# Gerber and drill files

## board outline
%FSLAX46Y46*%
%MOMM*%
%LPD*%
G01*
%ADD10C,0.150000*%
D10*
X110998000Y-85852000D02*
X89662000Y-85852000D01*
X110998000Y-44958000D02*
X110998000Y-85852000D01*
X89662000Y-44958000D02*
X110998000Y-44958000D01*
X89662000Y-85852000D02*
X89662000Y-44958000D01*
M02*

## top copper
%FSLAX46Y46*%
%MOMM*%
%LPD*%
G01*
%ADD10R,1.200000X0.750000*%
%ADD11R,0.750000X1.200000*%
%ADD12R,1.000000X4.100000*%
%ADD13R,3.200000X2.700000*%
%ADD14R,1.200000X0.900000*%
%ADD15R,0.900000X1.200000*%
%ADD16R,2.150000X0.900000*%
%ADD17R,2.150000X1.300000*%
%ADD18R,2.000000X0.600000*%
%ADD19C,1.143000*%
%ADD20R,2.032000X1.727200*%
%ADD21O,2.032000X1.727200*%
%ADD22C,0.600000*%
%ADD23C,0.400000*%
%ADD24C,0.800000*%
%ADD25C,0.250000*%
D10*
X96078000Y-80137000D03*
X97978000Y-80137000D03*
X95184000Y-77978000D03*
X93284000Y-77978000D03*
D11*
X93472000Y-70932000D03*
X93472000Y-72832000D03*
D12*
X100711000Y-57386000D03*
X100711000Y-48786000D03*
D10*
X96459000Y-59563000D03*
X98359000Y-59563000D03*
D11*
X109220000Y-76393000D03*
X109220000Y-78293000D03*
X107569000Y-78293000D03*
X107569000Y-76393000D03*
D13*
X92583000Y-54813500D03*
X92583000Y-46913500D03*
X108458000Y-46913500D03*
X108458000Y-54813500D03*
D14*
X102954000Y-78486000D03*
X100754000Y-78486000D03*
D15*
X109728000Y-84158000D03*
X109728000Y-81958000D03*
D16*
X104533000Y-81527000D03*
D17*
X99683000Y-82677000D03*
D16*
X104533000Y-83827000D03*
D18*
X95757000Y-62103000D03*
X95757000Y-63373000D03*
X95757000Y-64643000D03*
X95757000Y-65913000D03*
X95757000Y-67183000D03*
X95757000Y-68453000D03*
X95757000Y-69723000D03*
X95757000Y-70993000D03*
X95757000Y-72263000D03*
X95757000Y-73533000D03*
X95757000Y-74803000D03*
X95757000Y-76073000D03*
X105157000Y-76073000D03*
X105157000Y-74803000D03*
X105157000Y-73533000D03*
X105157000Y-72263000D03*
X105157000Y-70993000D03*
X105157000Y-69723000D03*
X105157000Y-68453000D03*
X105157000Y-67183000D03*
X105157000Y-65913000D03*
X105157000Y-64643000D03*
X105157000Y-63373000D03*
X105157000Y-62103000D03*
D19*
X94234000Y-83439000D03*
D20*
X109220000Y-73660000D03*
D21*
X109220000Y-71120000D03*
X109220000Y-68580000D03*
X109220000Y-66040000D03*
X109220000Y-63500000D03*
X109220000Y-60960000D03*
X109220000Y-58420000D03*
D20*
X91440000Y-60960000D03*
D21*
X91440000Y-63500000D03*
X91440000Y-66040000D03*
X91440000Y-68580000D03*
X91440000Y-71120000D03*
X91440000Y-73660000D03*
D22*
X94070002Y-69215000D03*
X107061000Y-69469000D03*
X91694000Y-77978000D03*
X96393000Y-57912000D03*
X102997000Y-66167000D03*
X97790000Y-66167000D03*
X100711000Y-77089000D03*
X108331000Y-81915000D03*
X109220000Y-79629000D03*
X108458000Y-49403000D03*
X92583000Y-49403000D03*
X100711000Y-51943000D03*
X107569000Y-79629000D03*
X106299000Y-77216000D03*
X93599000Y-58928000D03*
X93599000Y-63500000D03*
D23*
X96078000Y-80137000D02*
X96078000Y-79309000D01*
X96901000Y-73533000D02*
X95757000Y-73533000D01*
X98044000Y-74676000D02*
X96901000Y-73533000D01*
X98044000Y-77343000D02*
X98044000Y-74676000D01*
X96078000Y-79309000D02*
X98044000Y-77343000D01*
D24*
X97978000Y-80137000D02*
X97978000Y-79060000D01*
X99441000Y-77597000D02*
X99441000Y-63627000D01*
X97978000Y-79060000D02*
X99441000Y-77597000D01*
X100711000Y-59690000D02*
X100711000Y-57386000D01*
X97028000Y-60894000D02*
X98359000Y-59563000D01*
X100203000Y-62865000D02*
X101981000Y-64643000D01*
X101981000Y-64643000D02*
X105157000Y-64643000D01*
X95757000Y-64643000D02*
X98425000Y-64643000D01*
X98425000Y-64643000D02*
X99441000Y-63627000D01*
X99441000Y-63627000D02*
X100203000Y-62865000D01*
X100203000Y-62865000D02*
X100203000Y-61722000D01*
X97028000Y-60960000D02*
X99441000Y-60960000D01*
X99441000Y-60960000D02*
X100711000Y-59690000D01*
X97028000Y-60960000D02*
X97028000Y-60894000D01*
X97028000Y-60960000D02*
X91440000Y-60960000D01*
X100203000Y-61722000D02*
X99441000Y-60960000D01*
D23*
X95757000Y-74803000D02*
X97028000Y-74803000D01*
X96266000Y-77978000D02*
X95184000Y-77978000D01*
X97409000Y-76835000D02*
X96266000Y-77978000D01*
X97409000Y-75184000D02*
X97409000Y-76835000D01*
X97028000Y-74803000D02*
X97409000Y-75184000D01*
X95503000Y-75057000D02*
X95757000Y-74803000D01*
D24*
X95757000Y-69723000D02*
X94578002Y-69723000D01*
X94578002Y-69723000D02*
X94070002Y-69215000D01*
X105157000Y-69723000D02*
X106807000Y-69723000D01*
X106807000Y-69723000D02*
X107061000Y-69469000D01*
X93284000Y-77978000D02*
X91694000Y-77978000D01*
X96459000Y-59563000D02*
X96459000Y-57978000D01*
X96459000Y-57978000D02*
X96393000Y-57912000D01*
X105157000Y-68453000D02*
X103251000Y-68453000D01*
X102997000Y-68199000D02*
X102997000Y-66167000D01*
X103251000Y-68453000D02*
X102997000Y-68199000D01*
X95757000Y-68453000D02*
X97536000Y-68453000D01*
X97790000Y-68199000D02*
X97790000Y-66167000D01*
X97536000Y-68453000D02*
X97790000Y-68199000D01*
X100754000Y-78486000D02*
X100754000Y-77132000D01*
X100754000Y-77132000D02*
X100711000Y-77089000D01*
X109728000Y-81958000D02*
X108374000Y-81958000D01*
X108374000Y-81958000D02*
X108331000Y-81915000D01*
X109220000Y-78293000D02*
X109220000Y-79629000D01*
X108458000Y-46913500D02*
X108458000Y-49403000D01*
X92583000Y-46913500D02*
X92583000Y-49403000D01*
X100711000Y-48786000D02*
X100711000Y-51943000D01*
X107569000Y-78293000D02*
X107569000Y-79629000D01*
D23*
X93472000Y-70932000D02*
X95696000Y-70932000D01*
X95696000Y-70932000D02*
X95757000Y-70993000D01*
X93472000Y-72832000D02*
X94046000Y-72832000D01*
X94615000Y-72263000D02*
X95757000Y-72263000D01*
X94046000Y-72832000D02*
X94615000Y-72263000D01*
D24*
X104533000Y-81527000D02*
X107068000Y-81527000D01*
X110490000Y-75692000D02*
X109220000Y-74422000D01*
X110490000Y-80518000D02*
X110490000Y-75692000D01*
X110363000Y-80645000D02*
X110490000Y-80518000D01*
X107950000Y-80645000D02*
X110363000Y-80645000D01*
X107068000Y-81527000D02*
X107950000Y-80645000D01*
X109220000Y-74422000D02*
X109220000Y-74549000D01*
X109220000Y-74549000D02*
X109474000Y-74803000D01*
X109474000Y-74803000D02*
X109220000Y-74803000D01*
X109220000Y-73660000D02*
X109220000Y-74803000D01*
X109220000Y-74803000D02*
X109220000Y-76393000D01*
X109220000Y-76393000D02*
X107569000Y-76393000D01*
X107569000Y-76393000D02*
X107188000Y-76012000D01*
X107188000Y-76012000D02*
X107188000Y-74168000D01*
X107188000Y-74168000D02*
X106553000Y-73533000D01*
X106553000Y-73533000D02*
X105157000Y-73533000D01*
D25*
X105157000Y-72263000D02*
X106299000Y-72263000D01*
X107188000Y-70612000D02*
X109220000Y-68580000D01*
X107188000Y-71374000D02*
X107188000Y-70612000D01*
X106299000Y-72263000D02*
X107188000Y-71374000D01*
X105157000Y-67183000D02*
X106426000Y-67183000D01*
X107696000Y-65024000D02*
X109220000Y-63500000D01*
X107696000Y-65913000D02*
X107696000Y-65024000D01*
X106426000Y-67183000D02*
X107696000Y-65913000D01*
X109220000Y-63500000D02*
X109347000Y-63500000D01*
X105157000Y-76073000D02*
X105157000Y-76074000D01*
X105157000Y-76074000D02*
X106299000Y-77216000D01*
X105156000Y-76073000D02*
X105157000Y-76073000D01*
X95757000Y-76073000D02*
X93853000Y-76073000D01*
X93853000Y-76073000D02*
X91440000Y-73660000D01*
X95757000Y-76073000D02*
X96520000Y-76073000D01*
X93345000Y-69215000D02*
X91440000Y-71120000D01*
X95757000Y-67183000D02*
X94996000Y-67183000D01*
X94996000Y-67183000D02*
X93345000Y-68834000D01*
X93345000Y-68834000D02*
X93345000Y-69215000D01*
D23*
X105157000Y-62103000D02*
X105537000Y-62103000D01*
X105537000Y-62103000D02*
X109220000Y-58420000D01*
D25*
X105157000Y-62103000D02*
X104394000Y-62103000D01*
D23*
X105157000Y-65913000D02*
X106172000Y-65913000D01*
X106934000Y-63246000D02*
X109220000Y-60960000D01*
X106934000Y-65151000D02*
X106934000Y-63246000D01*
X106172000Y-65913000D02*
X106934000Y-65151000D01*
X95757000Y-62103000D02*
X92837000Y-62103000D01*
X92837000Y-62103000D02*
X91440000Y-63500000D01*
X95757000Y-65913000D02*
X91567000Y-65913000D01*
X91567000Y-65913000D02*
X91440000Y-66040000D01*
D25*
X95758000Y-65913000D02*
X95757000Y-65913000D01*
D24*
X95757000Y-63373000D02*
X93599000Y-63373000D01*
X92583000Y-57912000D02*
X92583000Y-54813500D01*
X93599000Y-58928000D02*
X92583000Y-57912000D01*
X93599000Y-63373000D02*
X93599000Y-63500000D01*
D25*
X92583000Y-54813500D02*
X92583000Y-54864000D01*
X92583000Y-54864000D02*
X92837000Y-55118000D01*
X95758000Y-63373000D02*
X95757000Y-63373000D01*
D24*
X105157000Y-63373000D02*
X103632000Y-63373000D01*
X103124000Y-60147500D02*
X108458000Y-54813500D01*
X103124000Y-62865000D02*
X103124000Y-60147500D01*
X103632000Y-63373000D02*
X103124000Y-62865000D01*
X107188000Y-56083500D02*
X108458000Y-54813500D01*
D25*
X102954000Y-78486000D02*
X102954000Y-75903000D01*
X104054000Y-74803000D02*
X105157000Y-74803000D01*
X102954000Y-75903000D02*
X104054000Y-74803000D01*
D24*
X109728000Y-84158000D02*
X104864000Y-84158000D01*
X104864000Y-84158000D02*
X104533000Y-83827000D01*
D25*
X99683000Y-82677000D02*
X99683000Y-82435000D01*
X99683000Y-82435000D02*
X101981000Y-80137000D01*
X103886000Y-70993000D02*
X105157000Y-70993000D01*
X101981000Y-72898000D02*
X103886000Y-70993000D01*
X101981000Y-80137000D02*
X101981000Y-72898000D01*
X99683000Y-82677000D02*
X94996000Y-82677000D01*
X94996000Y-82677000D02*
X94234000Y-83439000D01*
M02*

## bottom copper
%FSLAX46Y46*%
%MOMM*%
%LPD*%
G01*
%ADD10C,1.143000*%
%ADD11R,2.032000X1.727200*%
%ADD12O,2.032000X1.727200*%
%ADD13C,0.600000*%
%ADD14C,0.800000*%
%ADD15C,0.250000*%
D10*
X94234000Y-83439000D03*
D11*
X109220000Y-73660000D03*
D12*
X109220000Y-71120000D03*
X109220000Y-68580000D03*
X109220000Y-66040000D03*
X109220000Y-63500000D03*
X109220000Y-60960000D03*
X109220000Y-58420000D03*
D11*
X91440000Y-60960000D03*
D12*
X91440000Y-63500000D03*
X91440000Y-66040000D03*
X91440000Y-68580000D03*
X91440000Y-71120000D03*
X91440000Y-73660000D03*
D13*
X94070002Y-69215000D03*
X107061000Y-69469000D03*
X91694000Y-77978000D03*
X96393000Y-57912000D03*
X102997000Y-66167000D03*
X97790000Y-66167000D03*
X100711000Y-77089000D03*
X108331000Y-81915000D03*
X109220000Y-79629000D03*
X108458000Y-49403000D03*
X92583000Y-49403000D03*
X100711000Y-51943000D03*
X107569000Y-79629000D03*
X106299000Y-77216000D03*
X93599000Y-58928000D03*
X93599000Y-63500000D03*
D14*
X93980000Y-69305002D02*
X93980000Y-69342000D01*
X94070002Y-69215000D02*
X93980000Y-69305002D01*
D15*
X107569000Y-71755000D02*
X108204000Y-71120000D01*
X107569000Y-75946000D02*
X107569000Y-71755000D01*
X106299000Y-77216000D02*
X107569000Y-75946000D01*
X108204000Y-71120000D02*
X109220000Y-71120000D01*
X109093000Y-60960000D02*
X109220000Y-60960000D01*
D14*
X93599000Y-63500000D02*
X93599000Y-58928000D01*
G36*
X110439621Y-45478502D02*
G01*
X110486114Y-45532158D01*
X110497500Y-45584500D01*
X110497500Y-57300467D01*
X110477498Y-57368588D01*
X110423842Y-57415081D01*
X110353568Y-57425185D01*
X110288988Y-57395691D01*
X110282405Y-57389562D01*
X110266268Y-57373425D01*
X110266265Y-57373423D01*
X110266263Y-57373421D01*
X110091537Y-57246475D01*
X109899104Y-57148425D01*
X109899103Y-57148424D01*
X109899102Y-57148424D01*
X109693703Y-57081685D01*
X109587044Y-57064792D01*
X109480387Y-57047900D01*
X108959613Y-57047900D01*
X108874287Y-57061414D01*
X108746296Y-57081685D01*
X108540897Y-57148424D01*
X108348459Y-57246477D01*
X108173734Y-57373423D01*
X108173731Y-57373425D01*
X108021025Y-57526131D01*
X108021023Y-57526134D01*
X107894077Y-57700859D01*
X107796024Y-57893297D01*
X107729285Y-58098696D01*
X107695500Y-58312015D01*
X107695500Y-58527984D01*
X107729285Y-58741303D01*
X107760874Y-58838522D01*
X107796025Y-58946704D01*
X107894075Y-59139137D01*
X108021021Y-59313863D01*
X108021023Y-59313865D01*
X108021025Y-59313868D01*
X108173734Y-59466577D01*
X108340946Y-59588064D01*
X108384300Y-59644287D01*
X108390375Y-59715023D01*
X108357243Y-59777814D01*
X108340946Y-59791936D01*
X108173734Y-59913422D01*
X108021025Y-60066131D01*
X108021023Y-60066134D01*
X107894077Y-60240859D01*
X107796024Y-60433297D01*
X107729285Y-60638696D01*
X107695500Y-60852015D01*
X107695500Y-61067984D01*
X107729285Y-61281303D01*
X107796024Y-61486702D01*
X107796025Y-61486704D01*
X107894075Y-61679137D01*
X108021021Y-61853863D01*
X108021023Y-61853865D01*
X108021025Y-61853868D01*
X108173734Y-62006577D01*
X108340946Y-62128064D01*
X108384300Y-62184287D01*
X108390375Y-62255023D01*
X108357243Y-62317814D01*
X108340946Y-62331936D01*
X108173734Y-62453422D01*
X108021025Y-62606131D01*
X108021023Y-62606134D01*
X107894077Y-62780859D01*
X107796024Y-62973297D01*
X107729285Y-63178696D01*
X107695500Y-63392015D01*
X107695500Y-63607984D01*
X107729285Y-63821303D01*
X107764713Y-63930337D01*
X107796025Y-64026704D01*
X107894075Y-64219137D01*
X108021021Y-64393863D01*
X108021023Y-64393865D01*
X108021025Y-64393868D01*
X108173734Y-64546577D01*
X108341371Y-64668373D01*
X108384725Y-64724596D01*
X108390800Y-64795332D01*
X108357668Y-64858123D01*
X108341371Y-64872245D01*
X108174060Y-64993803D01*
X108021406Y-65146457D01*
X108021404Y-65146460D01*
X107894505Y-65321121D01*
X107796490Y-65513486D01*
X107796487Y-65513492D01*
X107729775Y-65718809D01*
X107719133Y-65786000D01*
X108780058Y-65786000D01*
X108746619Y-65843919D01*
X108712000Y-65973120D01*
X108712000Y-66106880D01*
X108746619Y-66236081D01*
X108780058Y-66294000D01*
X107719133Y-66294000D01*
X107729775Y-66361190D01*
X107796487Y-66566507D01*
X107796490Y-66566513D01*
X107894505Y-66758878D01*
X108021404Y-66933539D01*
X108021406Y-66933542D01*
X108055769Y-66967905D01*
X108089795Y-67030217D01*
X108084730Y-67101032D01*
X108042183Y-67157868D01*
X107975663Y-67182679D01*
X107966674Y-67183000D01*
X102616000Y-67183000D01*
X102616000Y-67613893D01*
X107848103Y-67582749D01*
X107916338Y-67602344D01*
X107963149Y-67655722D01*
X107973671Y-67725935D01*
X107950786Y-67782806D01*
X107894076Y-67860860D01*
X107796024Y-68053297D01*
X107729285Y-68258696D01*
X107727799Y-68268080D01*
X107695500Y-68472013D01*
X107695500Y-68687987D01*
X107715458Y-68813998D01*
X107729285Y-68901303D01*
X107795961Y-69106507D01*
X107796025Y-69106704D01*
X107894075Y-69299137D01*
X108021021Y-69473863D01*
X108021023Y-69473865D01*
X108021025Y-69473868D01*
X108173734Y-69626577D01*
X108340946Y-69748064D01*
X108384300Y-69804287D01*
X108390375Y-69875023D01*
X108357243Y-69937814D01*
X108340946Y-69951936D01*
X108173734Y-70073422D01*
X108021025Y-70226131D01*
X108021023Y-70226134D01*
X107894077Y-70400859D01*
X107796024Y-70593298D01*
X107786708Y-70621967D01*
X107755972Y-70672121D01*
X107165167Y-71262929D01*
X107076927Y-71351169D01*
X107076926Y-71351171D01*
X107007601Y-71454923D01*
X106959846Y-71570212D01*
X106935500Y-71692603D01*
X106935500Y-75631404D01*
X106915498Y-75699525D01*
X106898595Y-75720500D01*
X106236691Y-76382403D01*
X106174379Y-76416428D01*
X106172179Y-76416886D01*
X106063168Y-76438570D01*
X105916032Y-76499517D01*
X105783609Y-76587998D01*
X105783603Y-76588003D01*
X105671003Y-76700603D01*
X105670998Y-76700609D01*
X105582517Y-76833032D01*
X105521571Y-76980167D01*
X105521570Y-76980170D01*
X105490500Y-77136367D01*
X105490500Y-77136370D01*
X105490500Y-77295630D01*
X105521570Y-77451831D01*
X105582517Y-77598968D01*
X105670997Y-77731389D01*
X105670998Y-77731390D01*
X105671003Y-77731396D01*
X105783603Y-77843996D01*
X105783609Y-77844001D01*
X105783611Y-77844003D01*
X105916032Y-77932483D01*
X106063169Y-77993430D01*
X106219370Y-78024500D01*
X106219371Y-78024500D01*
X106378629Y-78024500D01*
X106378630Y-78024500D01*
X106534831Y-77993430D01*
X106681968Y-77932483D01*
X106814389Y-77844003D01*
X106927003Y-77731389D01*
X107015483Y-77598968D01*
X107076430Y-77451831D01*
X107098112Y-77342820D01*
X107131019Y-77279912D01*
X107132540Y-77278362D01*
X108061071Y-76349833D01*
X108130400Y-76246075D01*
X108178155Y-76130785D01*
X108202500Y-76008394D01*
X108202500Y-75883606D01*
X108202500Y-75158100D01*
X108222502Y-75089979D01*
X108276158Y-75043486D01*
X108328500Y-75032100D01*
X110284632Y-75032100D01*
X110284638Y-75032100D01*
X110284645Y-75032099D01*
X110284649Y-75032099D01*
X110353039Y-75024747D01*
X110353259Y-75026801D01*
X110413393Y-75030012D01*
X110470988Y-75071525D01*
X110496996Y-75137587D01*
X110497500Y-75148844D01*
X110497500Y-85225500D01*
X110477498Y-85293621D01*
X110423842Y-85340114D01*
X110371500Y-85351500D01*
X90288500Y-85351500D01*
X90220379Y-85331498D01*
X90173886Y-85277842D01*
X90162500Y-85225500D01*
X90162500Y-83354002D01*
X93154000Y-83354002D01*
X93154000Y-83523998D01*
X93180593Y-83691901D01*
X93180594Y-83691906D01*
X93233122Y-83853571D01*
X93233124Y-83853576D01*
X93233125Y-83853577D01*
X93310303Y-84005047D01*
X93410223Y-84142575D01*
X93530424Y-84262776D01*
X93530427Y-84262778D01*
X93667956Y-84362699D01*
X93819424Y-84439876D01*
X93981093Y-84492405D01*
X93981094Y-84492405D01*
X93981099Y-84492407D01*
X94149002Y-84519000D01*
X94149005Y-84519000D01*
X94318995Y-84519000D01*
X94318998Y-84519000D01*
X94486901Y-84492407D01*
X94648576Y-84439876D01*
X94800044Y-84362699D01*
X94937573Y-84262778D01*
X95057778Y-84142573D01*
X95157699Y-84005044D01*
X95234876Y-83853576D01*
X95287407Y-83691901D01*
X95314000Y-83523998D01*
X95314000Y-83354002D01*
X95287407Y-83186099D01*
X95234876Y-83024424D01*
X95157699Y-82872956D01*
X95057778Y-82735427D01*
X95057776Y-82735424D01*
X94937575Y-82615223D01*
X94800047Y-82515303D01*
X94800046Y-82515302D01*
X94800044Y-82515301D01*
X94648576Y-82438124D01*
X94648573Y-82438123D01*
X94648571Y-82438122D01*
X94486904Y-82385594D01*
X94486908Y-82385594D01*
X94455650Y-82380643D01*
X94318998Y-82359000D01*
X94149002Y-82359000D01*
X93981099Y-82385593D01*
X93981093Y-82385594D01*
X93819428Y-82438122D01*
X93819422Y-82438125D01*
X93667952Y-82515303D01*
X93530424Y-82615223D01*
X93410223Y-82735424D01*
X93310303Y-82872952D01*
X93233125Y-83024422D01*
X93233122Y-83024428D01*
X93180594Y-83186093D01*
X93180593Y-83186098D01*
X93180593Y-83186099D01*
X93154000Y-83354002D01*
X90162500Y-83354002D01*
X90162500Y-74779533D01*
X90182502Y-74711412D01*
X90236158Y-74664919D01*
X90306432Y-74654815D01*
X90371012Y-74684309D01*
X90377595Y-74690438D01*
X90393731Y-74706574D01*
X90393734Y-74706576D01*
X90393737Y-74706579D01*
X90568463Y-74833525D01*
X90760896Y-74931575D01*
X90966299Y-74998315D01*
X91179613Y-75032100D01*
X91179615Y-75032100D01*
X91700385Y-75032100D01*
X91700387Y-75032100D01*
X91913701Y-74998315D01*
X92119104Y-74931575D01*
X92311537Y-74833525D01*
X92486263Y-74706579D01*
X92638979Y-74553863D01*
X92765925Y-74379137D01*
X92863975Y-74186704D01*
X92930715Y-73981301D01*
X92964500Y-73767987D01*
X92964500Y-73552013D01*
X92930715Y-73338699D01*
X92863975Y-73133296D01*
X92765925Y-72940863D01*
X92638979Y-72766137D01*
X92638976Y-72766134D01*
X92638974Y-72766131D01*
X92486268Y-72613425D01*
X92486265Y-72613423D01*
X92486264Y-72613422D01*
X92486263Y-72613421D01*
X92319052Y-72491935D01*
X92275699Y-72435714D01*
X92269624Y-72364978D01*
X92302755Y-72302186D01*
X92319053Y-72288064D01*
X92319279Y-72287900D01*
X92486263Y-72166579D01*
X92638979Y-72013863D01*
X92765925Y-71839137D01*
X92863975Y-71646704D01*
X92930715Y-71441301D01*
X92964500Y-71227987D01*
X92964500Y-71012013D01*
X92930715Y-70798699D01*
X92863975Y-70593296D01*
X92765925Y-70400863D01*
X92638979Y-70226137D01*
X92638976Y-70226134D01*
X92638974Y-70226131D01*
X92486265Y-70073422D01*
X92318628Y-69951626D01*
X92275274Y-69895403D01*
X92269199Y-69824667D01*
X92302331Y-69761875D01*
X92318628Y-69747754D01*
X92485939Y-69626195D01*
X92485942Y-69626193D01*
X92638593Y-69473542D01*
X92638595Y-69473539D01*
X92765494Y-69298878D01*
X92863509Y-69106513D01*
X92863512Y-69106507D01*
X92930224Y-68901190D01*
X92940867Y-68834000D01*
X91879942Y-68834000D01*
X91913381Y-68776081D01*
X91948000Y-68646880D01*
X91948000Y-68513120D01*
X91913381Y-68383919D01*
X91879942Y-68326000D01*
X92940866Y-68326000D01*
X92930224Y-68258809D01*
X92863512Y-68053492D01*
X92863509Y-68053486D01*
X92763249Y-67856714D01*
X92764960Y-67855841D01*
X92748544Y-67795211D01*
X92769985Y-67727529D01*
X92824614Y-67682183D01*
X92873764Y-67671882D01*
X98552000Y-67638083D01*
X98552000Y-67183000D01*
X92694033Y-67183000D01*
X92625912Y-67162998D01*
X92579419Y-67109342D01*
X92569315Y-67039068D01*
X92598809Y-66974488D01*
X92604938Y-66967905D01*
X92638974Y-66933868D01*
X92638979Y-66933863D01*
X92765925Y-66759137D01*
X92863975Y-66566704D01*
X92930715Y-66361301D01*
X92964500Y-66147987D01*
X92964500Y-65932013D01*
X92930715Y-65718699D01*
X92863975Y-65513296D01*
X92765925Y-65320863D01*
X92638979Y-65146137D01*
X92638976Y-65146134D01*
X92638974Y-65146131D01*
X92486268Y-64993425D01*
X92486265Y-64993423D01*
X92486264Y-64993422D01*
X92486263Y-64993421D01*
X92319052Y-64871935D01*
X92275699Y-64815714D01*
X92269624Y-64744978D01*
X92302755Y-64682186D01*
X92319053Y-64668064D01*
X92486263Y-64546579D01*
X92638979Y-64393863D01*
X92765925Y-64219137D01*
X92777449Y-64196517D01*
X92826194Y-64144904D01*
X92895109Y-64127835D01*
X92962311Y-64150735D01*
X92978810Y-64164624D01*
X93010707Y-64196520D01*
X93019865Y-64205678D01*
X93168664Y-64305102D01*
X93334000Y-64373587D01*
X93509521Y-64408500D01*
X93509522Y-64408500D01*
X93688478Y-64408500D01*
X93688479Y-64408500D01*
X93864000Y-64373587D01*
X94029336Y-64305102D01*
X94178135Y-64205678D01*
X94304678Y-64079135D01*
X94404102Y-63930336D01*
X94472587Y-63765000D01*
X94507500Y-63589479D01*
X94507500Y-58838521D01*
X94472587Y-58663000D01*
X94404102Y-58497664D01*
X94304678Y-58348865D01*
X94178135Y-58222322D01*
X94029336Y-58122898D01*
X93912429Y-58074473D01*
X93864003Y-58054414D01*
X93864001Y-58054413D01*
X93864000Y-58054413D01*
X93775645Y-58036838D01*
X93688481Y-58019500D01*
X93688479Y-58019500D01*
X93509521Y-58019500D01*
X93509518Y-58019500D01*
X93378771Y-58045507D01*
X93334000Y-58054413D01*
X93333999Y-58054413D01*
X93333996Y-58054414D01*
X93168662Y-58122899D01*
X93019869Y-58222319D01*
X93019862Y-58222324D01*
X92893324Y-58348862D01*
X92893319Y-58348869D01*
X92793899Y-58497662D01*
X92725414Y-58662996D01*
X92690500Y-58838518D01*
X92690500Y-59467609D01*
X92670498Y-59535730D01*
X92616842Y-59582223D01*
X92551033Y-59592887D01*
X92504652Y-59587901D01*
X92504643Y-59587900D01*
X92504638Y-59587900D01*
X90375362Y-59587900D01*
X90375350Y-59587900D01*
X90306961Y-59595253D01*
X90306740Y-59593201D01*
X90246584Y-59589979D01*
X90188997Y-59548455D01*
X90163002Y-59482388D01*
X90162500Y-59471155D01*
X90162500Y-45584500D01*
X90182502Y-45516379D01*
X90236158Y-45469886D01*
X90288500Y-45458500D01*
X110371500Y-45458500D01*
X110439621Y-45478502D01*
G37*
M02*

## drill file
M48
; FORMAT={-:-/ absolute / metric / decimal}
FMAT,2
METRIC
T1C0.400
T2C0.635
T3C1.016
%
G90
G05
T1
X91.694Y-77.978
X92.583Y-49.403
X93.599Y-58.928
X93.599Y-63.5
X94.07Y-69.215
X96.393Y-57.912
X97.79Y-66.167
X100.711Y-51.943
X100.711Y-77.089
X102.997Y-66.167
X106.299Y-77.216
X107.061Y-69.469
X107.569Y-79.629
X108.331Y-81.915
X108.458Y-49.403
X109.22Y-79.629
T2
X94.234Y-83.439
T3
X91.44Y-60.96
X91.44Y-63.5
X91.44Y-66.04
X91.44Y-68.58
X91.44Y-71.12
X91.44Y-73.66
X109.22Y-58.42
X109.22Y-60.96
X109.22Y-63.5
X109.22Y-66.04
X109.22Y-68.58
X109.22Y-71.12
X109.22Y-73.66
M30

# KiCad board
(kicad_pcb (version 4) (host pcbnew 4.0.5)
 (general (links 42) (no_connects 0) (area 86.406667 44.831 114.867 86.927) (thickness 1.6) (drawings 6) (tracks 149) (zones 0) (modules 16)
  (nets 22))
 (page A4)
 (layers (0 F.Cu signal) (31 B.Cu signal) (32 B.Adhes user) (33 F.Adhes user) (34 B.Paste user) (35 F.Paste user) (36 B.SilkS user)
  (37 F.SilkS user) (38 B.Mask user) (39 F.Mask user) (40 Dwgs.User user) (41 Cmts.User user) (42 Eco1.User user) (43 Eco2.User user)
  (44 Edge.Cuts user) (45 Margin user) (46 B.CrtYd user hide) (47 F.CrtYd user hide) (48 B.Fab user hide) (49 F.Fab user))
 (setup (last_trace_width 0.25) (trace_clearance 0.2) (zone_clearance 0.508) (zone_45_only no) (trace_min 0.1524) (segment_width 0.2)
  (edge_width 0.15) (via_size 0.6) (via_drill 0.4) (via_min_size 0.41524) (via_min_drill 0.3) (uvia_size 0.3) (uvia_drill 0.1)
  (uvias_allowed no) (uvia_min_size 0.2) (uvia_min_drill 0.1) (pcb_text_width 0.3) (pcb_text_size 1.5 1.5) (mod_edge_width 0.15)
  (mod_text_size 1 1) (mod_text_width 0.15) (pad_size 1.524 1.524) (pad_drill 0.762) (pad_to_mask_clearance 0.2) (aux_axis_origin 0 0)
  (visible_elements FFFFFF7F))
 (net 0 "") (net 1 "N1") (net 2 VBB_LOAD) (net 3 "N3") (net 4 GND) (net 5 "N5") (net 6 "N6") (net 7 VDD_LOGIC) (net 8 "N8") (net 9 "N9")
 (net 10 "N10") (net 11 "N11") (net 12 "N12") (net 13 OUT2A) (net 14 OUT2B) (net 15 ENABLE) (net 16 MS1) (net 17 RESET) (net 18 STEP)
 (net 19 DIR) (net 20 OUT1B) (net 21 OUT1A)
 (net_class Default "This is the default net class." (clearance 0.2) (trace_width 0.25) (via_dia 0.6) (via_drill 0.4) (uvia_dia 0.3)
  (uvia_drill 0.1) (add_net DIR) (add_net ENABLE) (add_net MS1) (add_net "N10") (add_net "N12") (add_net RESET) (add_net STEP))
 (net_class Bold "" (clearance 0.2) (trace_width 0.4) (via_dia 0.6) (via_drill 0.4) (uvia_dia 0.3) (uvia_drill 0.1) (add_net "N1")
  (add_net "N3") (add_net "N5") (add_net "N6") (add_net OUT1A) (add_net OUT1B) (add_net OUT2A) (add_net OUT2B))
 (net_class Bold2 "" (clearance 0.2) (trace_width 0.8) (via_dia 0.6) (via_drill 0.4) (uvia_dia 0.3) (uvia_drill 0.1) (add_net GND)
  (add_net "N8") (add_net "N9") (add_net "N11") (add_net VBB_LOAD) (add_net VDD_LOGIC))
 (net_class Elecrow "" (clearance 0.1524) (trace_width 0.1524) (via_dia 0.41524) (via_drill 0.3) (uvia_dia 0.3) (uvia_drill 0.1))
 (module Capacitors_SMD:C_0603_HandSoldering (layer F.Cu) (at 97.028 80.137)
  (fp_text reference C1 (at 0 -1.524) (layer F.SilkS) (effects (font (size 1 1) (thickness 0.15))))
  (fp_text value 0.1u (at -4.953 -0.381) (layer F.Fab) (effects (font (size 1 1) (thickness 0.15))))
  (pad 1 smd rect (at -0.95 0) (size 1.2 0.75) (layers F.Cu F.Paste F.Mask) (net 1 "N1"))
  (pad 2 smd rect (at 0.95 0) (size 1.2 0.75) (layers F.Cu F.Paste F.Mask) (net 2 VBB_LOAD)))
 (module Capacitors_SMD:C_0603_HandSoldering (layer F.Cu) (at 94.234 77.978 180)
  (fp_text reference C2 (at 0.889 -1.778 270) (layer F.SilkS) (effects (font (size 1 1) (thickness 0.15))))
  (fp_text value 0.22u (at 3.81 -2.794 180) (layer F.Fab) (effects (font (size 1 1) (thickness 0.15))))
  (pad 1 smd rect (at -0.95 0 180) (size 1.2 0.75) (layers F.Cu F.Paste F.Mask) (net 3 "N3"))
  (pad 2 smd rect (at 0.95 0 180) (size 1.2 0.75) (layers F.Cu F.Paste F.Mask) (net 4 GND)))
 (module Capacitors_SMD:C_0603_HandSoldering (layer F.Cu) (at 93.472 71.882 270)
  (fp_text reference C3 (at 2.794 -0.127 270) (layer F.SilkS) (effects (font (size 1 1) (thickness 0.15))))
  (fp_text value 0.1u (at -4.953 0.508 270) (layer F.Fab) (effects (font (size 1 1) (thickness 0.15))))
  (pad 1 smd rect (at -0.95 0 270) (size 1.2 0.75) (layers F.Cu F.Paste F.Mask) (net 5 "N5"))
  (pad 2 smd rect (at 0.95 0 270) (size 1.2 0.75) (layers F.Cu F.Paste F.Mask) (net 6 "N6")))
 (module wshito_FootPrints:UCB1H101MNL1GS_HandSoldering (layer F.Cu) (at 100.711 53.086 180)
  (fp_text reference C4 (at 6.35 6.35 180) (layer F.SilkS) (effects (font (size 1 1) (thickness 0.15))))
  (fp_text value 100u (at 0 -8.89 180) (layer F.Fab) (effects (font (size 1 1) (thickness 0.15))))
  (pad 1 smd rect (at 0 -4.3 180) (size 1 4.1) (layers F.Cu F.Paste F.Mask) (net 2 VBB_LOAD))
  (pad 2 smd rect (at 0 4.3 180) (size 1 4.1) (layers F.Cu F.Paste F.Mask) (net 4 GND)))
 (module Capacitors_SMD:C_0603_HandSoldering (layer F.Cu) (at 97.409 59.563)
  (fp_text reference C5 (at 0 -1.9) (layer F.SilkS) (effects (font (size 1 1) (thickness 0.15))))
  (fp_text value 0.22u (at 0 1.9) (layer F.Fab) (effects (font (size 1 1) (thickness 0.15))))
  (pad 1 smd rect (at -0.95 0) (size 1.2 0.75) (layers F.Cu F.Paste F.Mask) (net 4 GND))
  (pad 2 smd rect (at 0.95 0) (size 1.2 0.75) (layers F.Cu F.Paste F.Mask) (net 2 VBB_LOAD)))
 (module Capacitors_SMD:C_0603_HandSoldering (layer F.Cu) (at 109.22 77.343 270)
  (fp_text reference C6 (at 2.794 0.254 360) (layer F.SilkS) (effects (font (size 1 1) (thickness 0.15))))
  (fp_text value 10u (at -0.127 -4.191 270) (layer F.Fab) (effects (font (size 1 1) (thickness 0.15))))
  (pad 1 smd rect (at -0.95 0 270) (size 1.2 0.75) (layers F.Cu F.Paste F.Mask) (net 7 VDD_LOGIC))
  (pad 2 smd rect (at 0.95 0 270) (size 1.2 0.75) (layers F.Cu F.Paste F.Mask) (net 4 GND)))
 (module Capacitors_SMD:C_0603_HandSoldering (layer F.Cu) (at 107.569 77.343 90)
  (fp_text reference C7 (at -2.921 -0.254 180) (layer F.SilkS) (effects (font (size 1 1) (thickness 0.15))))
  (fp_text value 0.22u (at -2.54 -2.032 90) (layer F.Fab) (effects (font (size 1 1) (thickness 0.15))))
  (pad 1 smd rect (at -0.95 0 90) (size 1.2 0.75) (layers F.Cu F.Paste F.Mask) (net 4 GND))
  (pad 2 smd rect (at 0.95 0 90) (size 1.2 0.75) (layers F.Cu F.Paste F.Mask) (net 7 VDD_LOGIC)))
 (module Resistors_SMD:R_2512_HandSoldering (layer F.Cu) (at 92.583 50.8635 90)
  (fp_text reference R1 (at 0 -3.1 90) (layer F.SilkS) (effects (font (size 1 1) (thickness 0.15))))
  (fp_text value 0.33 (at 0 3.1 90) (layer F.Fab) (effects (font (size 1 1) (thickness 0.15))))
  (pad 1 smd rect (at -3.95 0 90) (size 2.7 3.2) (layers F.Cu F.Paste F.Mask) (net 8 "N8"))
  (pad 2 smd rect (at 3.95 0 90) (size 2.7 3.2) (layers F.Cu F.Paste F.Mask) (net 4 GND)))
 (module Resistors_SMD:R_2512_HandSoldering (layer F.Cu) (at 108.458 50.8635 270)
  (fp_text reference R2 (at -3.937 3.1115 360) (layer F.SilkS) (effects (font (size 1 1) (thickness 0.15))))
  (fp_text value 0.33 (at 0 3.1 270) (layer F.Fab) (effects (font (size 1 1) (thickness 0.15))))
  (pad 1 smd rect (at -3.95 0 270) (size 2.7 3.2) (layers F.Cu F.Paste F.Mask) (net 4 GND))
  (pad 2 smd rect (at 3.95 0 270) (size 2.7 3.2) (layers F.Cu F.Paste F.Mask) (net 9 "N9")))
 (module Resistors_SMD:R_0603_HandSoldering (layer F.Cu) (at 101.854 78.486 180)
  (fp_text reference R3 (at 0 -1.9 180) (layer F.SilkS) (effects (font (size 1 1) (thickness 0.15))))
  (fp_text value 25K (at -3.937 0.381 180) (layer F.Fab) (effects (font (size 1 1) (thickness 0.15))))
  (pad 1 smd rect (at -1.1 0 180) (size 1.2 0.9) (layers F.Cu F.Paste F.Mask) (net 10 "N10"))
  (pad 2 smd rect (at 1.1 0 180) (size 1.2 0.9) (layers F.Cu F.Paste F.Mask) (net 4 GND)))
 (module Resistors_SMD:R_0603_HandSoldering (layer F.Cu) (at 109.728 83.058 90)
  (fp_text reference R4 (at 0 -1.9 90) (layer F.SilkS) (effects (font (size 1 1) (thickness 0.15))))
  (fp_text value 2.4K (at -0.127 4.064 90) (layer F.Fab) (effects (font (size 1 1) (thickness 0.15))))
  (pad 1 smd rect (at -1.1 0 90) (size 1.2 0.9) (layers F.Cu F.Paste F.Mask) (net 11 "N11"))
  (pad 2 smd rect (at 1.1 0 90) (size 1.2 0.9) (layers F.Cu F.Paste F.Mask) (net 4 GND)))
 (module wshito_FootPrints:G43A (layer F.Cu) (at 102.108 82.677 90)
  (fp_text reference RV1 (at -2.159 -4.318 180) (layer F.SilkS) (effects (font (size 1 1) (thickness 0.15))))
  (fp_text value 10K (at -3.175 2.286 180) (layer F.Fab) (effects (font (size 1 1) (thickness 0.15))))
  (pad 1 smd rect (at 1.15 2.425 90) (size 0.9 2.15) (layers F.Cu F.Paste F.Mask) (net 7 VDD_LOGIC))
  (pad 2 smd rect (at 0 -2.425 90) (size 1.3 2.15) (layers F.Cu F.Paste F.Mask) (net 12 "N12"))
  (pad 3 smd rect (at -1.15 2.425 90) (size 0.9 2.15) (layers F.Cu F.Paste F.Mask) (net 11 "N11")))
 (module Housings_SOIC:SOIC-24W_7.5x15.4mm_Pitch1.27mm (layer F.Cu) (at 100.457 69.088)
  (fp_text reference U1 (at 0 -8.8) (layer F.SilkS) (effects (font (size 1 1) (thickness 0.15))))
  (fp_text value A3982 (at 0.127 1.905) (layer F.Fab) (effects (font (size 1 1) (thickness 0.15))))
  (pad 1 smd rect (at -4.7 -6.985) (size 2 0.6) (layers F.Cu F.Paste F.Mask) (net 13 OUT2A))
  (pad 2 smd rect (at -4.7 -5.715) (size 2 0.6) (layers F.Cu F.Paste F.Mask) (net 8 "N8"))
  (pad 3 smd rect (at -4.7 -4.445) (size 2 0.6) (layers F.Cu F.Paste F.Mask) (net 2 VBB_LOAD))
  (pad 4 smd rect (at -4.7 -3.175) (size 2 0.6) (layers F.Cu F.Paste F.Mask) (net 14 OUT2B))
  (pad 5 smd rect (at -4.7 -1.905) (size 2 0.6) (layers F.Cu F.Paste F.Mask) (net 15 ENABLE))
  (pad 6 smd rect (at -4.7 -0.635) (size 2 0.6) (layers F.Cu F.Paste F.Mask) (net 4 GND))
  (pad 7 smd rect (at -4.7 0.635) (size 2 0.6) (layers F.Cu F.Paste F.Mask) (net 4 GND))
  (pad 8 smd rect (at -4.7 1.905) (size 2 0.6) (layers F.Cu F.Paste F.Mask) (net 5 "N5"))
  (pad 9 smd rect (at -4.7 3.175) (size 2 0.6) (layers F.Cu F.Paste F.Mask) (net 6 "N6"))
  (pad 10 smd rect (at -4.7 4.445) (size 2 0.6) (layers F.Cu F.Paste F.Mask) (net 1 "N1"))
  (pad 11 smd rect (at -4.7 5.715) (size 2 0.6) (layers F.Cu F.Paste F.Mask) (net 3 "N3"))
  (pad 12 smd rect (at -4.7 6.985) (size 2 0.6) (layers F.Cu F.Paste F.Mask) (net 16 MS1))
  (pad 13 smd rect (at 4.7 6.985) (size 2 0.6) (layers F.Cu F.Paste F.Mask) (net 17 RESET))
  (pad 14 smd rect (at 4.7 5.715) (size 2 0.6) (layers F.Cu F.Paste F.Mask) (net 10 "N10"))
  (pad 15 smd rect (at 4.7 4.445) (size 2 0.6) (layers F.Cu F.Paste F.Mask) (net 7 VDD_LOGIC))
  (pad 16 smd rect (at 4.7 3.175) (size 2 0.6) (layers F.Cu F.Paste F.Mask) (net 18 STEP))
  (pad 17 smd rect (at 4.7 1.905) (size 2 0.6) (layers F.Cu F.Paste F.Mask) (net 12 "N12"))
  (pad 18 smd rect (at 4.7 0.635) (size 2 0.6) (layers F.Cu F.Paste F.Mask) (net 4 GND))
  (pad 19 smd rect (at 4.7 -0.635) (size 2 0.6) (layers F.Cu F.Paste F.Mask) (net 4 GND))
  (pad 20 smd rect (at 4.7 -1.905) (size 2 0.6) (layers F.Cu F.Paste F.Mask) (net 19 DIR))
  (pad 21 smd rect (at 4.7 -3.175) (size 2 0.6) (layers F.Cu F.Paste F.Mask) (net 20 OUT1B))
  (pad 22 smd rect (at 4.7 -4.445) (size 2 0.6) (layers F.Cu F.Paste F.Mask) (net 2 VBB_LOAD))
  (pad 23 smd rect (at 4.7 -5.715) (size 2 0.6) (layers F.Cu F.Paste F.Mask) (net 9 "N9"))
  (pad 24 smd rect (at 4.7 -6.985) (size 2 0.6) (layers F.Cu F.Paste F.Mask) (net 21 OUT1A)))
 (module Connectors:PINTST (layer F.Cu) (at 94.234 83.439)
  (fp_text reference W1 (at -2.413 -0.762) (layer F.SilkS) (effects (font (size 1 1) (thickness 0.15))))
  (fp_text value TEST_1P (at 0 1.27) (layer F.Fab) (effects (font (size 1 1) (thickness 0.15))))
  (pad 1 thru_hole circle (at 0 0) (size 1.143 1.143) (drill 0.635) (layers *.Cu *.Mask) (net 12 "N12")))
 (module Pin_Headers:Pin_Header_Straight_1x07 (layer F.Cu) (at 109.22 73.66 180)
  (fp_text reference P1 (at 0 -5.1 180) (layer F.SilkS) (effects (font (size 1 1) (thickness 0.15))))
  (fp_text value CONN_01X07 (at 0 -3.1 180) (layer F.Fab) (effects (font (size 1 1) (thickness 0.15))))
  (pad 1 thru_hole rect (at 0 0 180) (size 2.032 1.7272) (drill 1.016) (layers *.Cu *.Mask) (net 7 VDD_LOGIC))
  (pad 2 thru_hole oval (at 0 2.54 180) (size 2.032 1.7272) (drill 1.016) (layers *.Cu *.Mask) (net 17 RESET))
  (pad 3 thru_hole oval (at 0 5.08 180) (size 2.032 1.7272) (drill 1.016) (layers *.Cu *.Mask) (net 18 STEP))
  (pad 4 thru_hole oval (at 0 7.62 180) (size 2.032 1.7272) (drill 1.016) (layers *.Cu *.Mask) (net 4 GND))
  (pad 5 thru_hole oval (at 0 10.16 180) (size 2.032 1.7272) (drill 1.016) (layers *.Cu *.Mask) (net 19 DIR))
  (pad 6 thru_hole oval (at 0 12.7 180) (size 2.032 1.7272) (drill 1.016) (layers *.Cu *.Mask) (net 20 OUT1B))
  (pad 7 thru_hole oval (at 0 15.24 180) (size 2.032 1.7272) (drill 1.016) (layers *.Cu *.Mask) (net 21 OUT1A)))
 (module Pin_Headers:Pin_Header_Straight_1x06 (layer F.Cu) (at 91.44 60.96)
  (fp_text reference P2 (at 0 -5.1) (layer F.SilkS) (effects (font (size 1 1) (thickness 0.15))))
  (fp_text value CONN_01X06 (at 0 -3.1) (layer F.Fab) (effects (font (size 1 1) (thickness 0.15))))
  (pad 1 thru_hole rect (at 0 0) (size 2.032 1.7272) (drill 1.016) (layers *.Cu *.Mask) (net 2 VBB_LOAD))
  (pad 2 thru_hole oval (at 0 2.54) (size 2.032 1.7272) (drill 1.016) (layers *.Cu *.Mask) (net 13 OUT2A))
  (pad 3 thru_hole oval (at 0 5.08) (size 2.032 1.7272) (drill 1.016) (layers *.Cu *.Mask) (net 14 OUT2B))
  (pad 4 thru_hole oval (at 0 7.62) (size 2.032 1.7272) (drill 1.016) (layers *.Cu *.Mask) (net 4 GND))
  (pad 5 thru_hole oval (at 0 10.16) (size 2.032 1.7272) (drill 1.016) (layers *.Cu *.Mask) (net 15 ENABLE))
  (pad 6 thru_hole oval (at 0 12.7) (size 2.032 1.7272) (drill 1.016) (layers *.Cu *.Mask) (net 16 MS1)))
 (gr_line (start 110.998 85.852) (end 89.662 85.852) (angle 90) (layer Edge.Cuts) (width 0.15))
 (gr_line (start 110.998 44.958) (end 110.998 85.852) (angle 90) (layer Edge.Cuts) (width 0.15))
 (gr_line (start 89.662 44.958) (end 110.998 44.958) (angle 90) (layer Edge.Cuts) (width 0.15))
 (gr_line (start 89.662 85.852) (end 89.662 44.958) (angle 90) (layer Edge.Cuts) (width 0.15))
 (segment (start 96.078 80.137) (end 96.078 79.309) (width 0.4) (layer F.Cu) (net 1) (status 10))
 (segment (start 96.901 73.533) (end 95.757 73.533) (width 0.4) (layer F.Cu) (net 1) (status 20))
 (segment (start 98.044 74.676) (end 96.901 73.533) (width 0.4) (layer F.Cu) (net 1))
 (segment (start 98.044 77.343) (end 98.044 74.676) (width 0.4) (layer F.Cu) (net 1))
 (segment (start 96.078 79.309) (end 98.044 77.343) (width 0.4) (layer F.Cu) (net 1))
 (segment (start 97.978 80.137) (end 97.978 79.06) (width 0.8) (layer F.Cu) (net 2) (status 10))
 (segment (start 99.441 77.597) (end 99.441 63.627) (width 0.8) (layer F.Cu) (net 2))
 (segment (start 97.978 79.06) (end 99.441 77.597) (width 0.8) (layer F.Cu) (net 2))
 (segment (start 100.711 59.69) (end 100.711 57.386) (width 0.8) (layer F.Cu) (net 2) (status 20))
 (segment (start 97.028 60.894) (end 98.359 59.563) (width 0.8) (layer F.Cu) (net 2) (status 20))
 (segment (start 100.203 62.865) (end 101.981 64.643) (width 0.8) (layer F.Cu) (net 2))
 (segment (start 101.981 64.643) (end 105.157 64.643) (width 0.8) (layer F.Cu) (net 2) (status 20))
 (segment (start 95.757 64.643) (end 98.425 64.643) (width 0.8) (layer F.Cu) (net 2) (status 10))
 (segment (start 98.425 64.643) (end 99.441 63.627) (width 0.8) (layer F.Cu) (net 2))
 (segment (start 99.441 63.627) (end 100.203 62.865) (width 0.8) (layer F.Cu) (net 2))
 (segment (start 100.203 62.865) (end 100.203 61.722) (width 0.8) (layer F.Cu) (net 2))
 (segment (start 97.028 60.96) (end 99.441 60.96) (width 0.8) (layer F.Cu) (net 2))
 (segment (start 99.441 60.96) (end 100.711 59.69) (width 0.8) (layer F.Cu) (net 2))
 (segment (start 97.028 60.96) (end 97.028 60.894) (width 0.8) (layer F.Cu) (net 2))
 (segment (start 97.028 60.96) (end 91.44 60.96) (width 0.8) (layer F.Cu) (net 2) (status 20))
 (segment (start 100.203 61.722) (end 99.441 60.96) (width 0.8) (layer F.Cu) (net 2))
 (segment (start 95.757 74.803) (end 97.028 74.803) (width 0.4) (layer F.Cu) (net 3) (status 10))
 (segment (start 96.266 77.978) (end 95.184 77.978) (width 0.4) (layer F.Cu) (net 3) (status 20))
 (segment (start 97.409 76.835) (end 96.266 77.978) (width 0.4) (layer F.Cu) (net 3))
 (segment (start 97.409 75.184) (end 97.409 76.835) (width 0.4) (layer F.Cu) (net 3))
 (segment (start 97.028 74.803) (end 97.409 75.184) (width 0.4) (layer F.Cu) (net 3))
 (segment (start 95.503 75.057) (end 95.757 74.803) (width 0.4) (layer F.Cu) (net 3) (status 30))
 (segment (start 95.757 69.723) (end 94.578002 69.723) (width 0.8) (layer F.Cu) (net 4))
 (segment (start 93.98 69.305002) (end 93.98 69.342) (width 0.8) (layer B.Cu) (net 4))
 (segment (start 94.070002 69.215) (end 93.98 69.305002) (width 0.8) (layer B.Cu) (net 4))
 (via (at 94.070002 69.215) (size 0.6) (drill 0.4) (layers F.Cu B.Cu) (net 4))
 (segment (start 94.578002 69.723) (end 94.070002 69.215) (width 0.8) (layer F.Cu) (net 4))
 (segment (start 105.157 69.723) (end 106.807 69.723) (width 0.8) (layer F.Cu) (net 4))
 (via (at 107.061 69.469) (size 0.6) (drill 0.4) (layers F.Cu B.Cu) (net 4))
 (segment (start 106.807 69.723) (end 107.061 69.469) (width 0.8) (layer F.Cu) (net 4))
 (segment (start 93.284 77.978) (end 91.694 77.978) (width 0.8) (layer F.Cu) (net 4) (status 10))
 (via (at 91.694 77.978) (size 0.6) (drill 0.4) (layers F.Cu B.Cu) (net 4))
 (segment (start 96.459 59.563) (end 96.459 57.978) (width 0.8) (layer F.Cu) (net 4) (status 10))
 (via (at 96.393 57.912) (size 0.6) (drill 0.4) (layers F.Cu B.Cu) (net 4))
 (segment (start 96.459 57.978) (end 96.393 57.912) (width 0.8) (layer F.Cu) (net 4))
 (segment (start 105.157 68.453) (end 103.251 68.453) (width 0.8) (layer F.Cu) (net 4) (status 10))
 (via (at 102.997 66.167) (size 0.6) (drill 0.4) (layers F.Cu B.Cu) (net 4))
 (segment (start 102.997 68.199) (end 102.997 66.167) (width 0.8) (layer F.Cu) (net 4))
 (segment (start 103.251 68.453) (end 102.997 68.199) (width 0.8) (layer F.Cu) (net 4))
 (segment (start 95.757 68.453) (end 97.536 68.453) (width 0.8) (layer F.Cu) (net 4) (status 10))
 (via (at 97.79 66.167) (size 0.6) (drill 0.4) (layers F.Cu B.Cu) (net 4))
 (segment (start 97.79 68.199) (end 97.79 66.167) (width 0.8) (layer F.Cu) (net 4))
 (segment (start 97.536 68.453) (end 97.79 68.199) (width 0.8) (layer F.Cu) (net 4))
 (segment (start 100.754 78.486) (end 100.754 77.132) (width 0.8) (layer F.Cu) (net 4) (status 10))
 (via (at 100.711 77.089) (size 0.6) (drill 0.4) (layers F.Cu B.Cu) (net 4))
 (segment (start 100.754 77.132) (end 100.711 77.089) (width 0.8) (layer F.Cu) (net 4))
 (segment (start 109.728 81.958) (end 108.374 81.958) (width 0.8) (layer F.Cu) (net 4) (status 10))
 (via (at 108.331 81.915) (size 0.6) (drill 0.4) (layers F.Cu B.Cu) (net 4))
 (segment (start 108.374 81.958) (end 108.331 81.915) (width 0.8) (layer F.Cu) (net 4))
 (segment (start 109.22 78.293) (end 109.22 79.629) (width 0.8) (layer F.Cu) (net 4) (status 10))
 (via (at 109.22 79.629) (size 0.6) (drill 0.4) (layers F.Cu B.Cu) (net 4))
 (segment (start 108.458 46.9135) (end 108.458 49.403) (width 0.8) (layer F.Cu) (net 4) (status 10))
 (via (at 108.458 49.403) (size 0.6) (drill 0.4) (layers F.Cu B.Cu) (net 4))
 (segment (start 92.583 46.9135) (end 92.583 49.403) (width 0.8) (layer F.Cu) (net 4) (status 10))
 (via (at 92.583 49.403) (size 0.6) (drill 0.4) (layers F.Cu B.Cu) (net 4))
 (segment (start 100.711 48.786) (end 100.711 51.943) (width 0.8) (layer F.Cu) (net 4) (status 10))
 (via (at 100.711 51.943) (size 0.6) (drill 0.4) (layers F.Cu B.Cu) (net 4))
 (segment (start 107.569 78.293) (end 107.569 79.629) (width 0.8) (layer F.Cu) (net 4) (status 10))
 (via (at 107.569 79.629) (size 0.6) (drill 0.4) (layers F.Cu B.Cu) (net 4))
 (segment (start 93.472 70.932) (end 95.696 70.932) (width 0.4) (layer F.Cu) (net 5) (status 30))
 (segment (start 95.696 70.932) (end 95.757 70.993) (width 0.4) (layer F.Cu) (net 5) (status 30))
 (segment (start 93.472 72.832) (end 94.046 72.832) (width 0.4) (layer F.Cu) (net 6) (status 10))
 (segment (start 94.615 72.263) (end 95.757 72.263) (width 0.4) (layer F.Cu) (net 6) (status 20))
 (segment (start 94.046 72.832) (end 94.615 72.263) (width 0.4) (layer F.Cu) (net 6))
 (segment (start 104.533 81.527) (end 107.068 81.527) (width 0.8) (layer F.Cu) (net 7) (status 10))
 (segment (start 110.49 75.692) (end 109.22 74.422) (width 0.8) (layer F.Cu) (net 7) (status 20))
 (segment (start 110.49 80.518) (end 110.49 75.692) (width 0.8) (layer F.Cu) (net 7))
 (segment (start 110.363 80.645) (end 110.49 80.518) (width 0.8) (layer F.Cu) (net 7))
 (segment (start 107.95 80.645) (end 110.363 80.645) (width 0.8) (layer F.Cu) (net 7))
 (segment (start 107.068 81.527) (end 107.95 80.645) (width 0.8) (layer F.Cu) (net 7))
 (segment (start 109.22 74.422) (end 109.22 74.549) (width 0.8) (layer F.Cu) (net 7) (status 10))
 (segment (start 109.22 74.549) (end 109.474 74.803) (width 0.8) (layer F.Cu) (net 7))
 (segment (start 109.474 74.803) (end 109.22 74.803) (width 0.8) (layer F.Cu) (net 7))
 (segment (start 109.22 73.66) (end 109.22 74.803) (width 0.8) (layer F.Cu) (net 7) (status 10))
 (segment (start 109.22 74.803) (end 109.22 76.393) (width 0.8) (layer F.Cu) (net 7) (status 20))
 (segment (start 109.22 76.393) (end 107.569 76.393) (width 0.8) (layer F.Cu) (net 7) (status 30))
 (segment (start 107.569 76.393) (end 107.188 76.012) (width 0.8) (layer F.Cu) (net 7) (status 10))
 (segment (start 107.188 76.012) (end 107.188 74.168) (width 0.8) (layer F.Cu) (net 7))
 (segment (start 107.188 74.168) (end 106.553 73.533) (width 0.8) (layer F.Cu) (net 7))
 (segment (start 106.553 73.533) (end 105.157 73.533) (width 0.8) (layer F.Cu) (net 7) (status 20))
 (segment (start 105.157 72.263) (end 106.299 72.263) (width 0.25) (layer F.Cu) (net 18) (status 10))
 (segment (start 107.188 70.612) (end 109.22 68.58) (width 0.25) (layer F.Cu) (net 18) (status 20))
 (segment (start 107.188 71.374) (end 107.188 70.612) (width 0.25) (layer F.Cu) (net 18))
 (segment (start 106.299 72.263) (end 107.188 71.374) (width 0.25) (layer F.Cu) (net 18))
 (segment (start 105.157 67.183) (end 106.426 67.183) (width 0.25) (layer F.Cu) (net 19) (status 10))
 (segment (start 107.696 65.024) (end 109.22 63.5) (width 0.25) (layer F.Cu) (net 19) (status 20))
 (segment (start 107.696 65.913) (end 107.696 65.024) (width 0.25) (layer F.Cu) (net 19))
 (segment (start 106.426 67.183) (end 107.696 65.913) (width 0.25) (layer F.Cu) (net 19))
 (segment (start 109.22 63.5) (end 109.347 63.5) (width 0.25) (layer F.Cu) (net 19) (status 80030))
 (segment (start 105.157 76.073) (end 105.157 76.074) (width 0.25) (layer F.Cu) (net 17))
 (segment (start 105.157 76.074) (end 106.299 77.216) (width 0.25) (layer F.Cu) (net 17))
 (segment (start 107.569 71.755) (end 108.204 71.12) (width 0.25) (layer B.Cu) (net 17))
 (segment (start 107.569 75.946) (end 107.569 71.755) (width 0.25) (layer B.Cu) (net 17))
 (segment (start 106.299 77.216) (end 107.569 75.946) (width 0.25) (layer B.Cu) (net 17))
 (via (at 106.299 77.216) (size 0.6) (drill 0.4) (layers F.Cu B.Cu) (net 17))
 (segment (start 108.204 71.12) (end 109.22 71.12) (width 0.25) (layer B.Cu) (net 17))
 (segment (start 105.156 76.073) (end 105.157 76.073) (width 0.25) (layer F.Cu) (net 17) (status 80030))
 (segment (start 95.757 76.073) (end 93.853 76.073) (width 0.25) (layer F.Cu) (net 16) (status 10))
 (segment (start 93.853 76.073) (end 91.44 73.66) (width 0.25) (layer F.Cu) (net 16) (status 20))
 (segment (start 95.757 76.073) (end 96.52 76.073) (width 0.25) (layer F.Cu) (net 16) (status 80030))
 (segment (start 93.345 69.215) (end 91.44 71.12) (width 0.25) (layer F.Cu) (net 15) (status 20))
 (segment (start 95.757 67.183) (end 94.996 67.183) (width 0.25) (layer F.Cu) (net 15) (status 30))
 (segment (start 94.996 67.183) (end 93.345 68.834) (width 0.25) (layer F.Cu) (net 15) (status 10))
 (segment (start 93.345 68.834) (end 93.345 69.215) (width 0.25) (layer F.Cu) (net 15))
 (segment (start 105.157 62.103) (end 105.537 62.103) (width 0.4) (layer F.Cu) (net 21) (status 30))
 (segment (start 105.537 62.103) (end 109.22 58.42) (width 0.4) (layer F.Cu) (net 21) (status 30))
 (segment (start 105.157 62.103) (end 104.394 62.103) (width 0.25) (layer F.Cu) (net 21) (status 80030))
 (segment (start 105.157 65.913) (end 106.172 65.913) (width 0.4) (layer F.Cu) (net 20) (status 10))
 (segment (start 106.934 63.246) (end 109.22 60.96) (width 0.4) (layer F.Cu) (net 20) (status 20))
 (segment (start 106.934 65.151) (end 106.934 63.246) (width 0.4) (layer F.Cu) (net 20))
 (segment (start 106.172 65.913) (end 106.934 65.151) (width 0.4) (layer F.Cu) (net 20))
 (segment (start 109.093 60.96) (end 109.22 60.96) (width 0.25) (layer B.Cu) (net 20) (status 80030))
 (segment (start 95.757 62.103) (end 92.837 62.103) (width 0.4) (layer F.Cu) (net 13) (status 10))
 (segment (start 92.837 62.103) (end 91.44 63.5) (width 0.4) (layer F.Cu) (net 13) (status 20))
 (segment (start 95.757 65.913) (end 91.567 65.913) (width 0.4) (layer F.Cu) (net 14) (status 30))
 (segment (start 91.567 65.913) (end 91.44 66.04) (width 0.4) (layer F.Cu) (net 14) (status 30))
 (segment (start 95.758 65.913) (end 95.757 65.913) (width 0.25) (layer F.Cu) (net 14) (status 80030))
 (segment (start 95.757 63.373) (end 93.599 63.373) (width 0.8) (layer F.Cu) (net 8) (status 10))
 (segment (start 92.583 57.912) (end 92.583 54.8135) (width 0.8) (layer F.Cu) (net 8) (status 20))
 (segment (start 93.599 58.928) (end 92.583 57.912) (width 0.8) (layer F.Cu) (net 8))
 (via (at 93.599 58.928) (size 0.6) (drill 0.4) (layers F.Cu B.Cu) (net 8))
 (segment (start 93.599 63.5) (end 93.599 58.928) (width 0.8) (layer B.Cu) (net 8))
 (via (at 93.599 63.5) (size 0.6) (drill 0.4) (layers F.Cu B.Cu) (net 8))
 (segment (start 93.599 63.373) (end 93.599 63.5) (width 0.8) (layer F.Cu) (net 8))
 (segment (start 92.583 54.8135) (end 92.583 54.864) (width 0.25) (layer F.Cu) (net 8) (status 80030))
 (segment (start 92.583 54.864) (end 92.837 55.118) (width 0.25) (layer F.Cu) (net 8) (status 80030))
 (segment (start 95.758 63.373) (end 95.757 63.373) (width 0.25) (layer F.Cu) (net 8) (status 80030))
 (segment (start 105.157 63.373) (end 103.632 63.373) (width 0.8) (layer F.Cu) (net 9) (status 10))
 (segment (start 103.124 60.1475) (end 108.458 54.8135) (width 0.8) (layer F.Cu) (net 9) (status 20))
 (segment (start 103.124 62.865) (end 103.124 60.1475) (width 0.8) (layer F.Cu) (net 9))
 (segment (start 103.632 63.373) (end 103.124 62.865) (width 0.8) (layer F.Cu) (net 9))
 (segment (start 107.188 56.0835) (end 108.458 54.8135) (width 0.8) (layer F.Cu) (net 9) (status 30))
 (segment (start 102.954 78.486) (end 102.954 75.903) (width 0.25) (layer F.Cu) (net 10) (status 10))
 (segment (start 104.054 74.803) (end 105.157 74.803) (width 0.25) (layer F.Cu) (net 10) (status 20))
 (segment (start 102.954 75.903) (end 104.054 74.803) (width 0.25) (layer F.Cu) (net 10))
 (segment (start 109.728 84.158) (end 104.864 84.158) (width 0.8) (layer F.Cu) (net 11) (status 30))
 (segment (start 104.864 84.158) (end 104.533 83.827) (width 0.8) (layer F.Cu) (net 11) (status 30))
 (segment (start 99.683 82.677) (end 99.683 82.435) (width 0.25) (layer F.Cu) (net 12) (status 30))
 (segment (start 99.683 82.435) (end 101.981 80.137) (width 0.25) (layer F.Cu) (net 12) (status 10))
 (segment (start 103.886 70.993) (end 105.157 70.993) (width 0.25) (layer F.Cu) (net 12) (status 20))
 (segment (start 101.981 72.898) (end 103.886 70.993) (width 0.25) (layer F.Cu) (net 12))
 (segment (start 101.981 80.137) (end 101.981 72.898) (width 0.25) (layer F.Cu) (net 12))
 (segment (start 99.683 82.677) (end 94.996 82.677) (width 0.25) (layer F.Cu) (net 12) (status 10))
 (segment (start 94.996 82.677) (end 94.234 83.439) (width 0.25) (layer F.Cu) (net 12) (status 20))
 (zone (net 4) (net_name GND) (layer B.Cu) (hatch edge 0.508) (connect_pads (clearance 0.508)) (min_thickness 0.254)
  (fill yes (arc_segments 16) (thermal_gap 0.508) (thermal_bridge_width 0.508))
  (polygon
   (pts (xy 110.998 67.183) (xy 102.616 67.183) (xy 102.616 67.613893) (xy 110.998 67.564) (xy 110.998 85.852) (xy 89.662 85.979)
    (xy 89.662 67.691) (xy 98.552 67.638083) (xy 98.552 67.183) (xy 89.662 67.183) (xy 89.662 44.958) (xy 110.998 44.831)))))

